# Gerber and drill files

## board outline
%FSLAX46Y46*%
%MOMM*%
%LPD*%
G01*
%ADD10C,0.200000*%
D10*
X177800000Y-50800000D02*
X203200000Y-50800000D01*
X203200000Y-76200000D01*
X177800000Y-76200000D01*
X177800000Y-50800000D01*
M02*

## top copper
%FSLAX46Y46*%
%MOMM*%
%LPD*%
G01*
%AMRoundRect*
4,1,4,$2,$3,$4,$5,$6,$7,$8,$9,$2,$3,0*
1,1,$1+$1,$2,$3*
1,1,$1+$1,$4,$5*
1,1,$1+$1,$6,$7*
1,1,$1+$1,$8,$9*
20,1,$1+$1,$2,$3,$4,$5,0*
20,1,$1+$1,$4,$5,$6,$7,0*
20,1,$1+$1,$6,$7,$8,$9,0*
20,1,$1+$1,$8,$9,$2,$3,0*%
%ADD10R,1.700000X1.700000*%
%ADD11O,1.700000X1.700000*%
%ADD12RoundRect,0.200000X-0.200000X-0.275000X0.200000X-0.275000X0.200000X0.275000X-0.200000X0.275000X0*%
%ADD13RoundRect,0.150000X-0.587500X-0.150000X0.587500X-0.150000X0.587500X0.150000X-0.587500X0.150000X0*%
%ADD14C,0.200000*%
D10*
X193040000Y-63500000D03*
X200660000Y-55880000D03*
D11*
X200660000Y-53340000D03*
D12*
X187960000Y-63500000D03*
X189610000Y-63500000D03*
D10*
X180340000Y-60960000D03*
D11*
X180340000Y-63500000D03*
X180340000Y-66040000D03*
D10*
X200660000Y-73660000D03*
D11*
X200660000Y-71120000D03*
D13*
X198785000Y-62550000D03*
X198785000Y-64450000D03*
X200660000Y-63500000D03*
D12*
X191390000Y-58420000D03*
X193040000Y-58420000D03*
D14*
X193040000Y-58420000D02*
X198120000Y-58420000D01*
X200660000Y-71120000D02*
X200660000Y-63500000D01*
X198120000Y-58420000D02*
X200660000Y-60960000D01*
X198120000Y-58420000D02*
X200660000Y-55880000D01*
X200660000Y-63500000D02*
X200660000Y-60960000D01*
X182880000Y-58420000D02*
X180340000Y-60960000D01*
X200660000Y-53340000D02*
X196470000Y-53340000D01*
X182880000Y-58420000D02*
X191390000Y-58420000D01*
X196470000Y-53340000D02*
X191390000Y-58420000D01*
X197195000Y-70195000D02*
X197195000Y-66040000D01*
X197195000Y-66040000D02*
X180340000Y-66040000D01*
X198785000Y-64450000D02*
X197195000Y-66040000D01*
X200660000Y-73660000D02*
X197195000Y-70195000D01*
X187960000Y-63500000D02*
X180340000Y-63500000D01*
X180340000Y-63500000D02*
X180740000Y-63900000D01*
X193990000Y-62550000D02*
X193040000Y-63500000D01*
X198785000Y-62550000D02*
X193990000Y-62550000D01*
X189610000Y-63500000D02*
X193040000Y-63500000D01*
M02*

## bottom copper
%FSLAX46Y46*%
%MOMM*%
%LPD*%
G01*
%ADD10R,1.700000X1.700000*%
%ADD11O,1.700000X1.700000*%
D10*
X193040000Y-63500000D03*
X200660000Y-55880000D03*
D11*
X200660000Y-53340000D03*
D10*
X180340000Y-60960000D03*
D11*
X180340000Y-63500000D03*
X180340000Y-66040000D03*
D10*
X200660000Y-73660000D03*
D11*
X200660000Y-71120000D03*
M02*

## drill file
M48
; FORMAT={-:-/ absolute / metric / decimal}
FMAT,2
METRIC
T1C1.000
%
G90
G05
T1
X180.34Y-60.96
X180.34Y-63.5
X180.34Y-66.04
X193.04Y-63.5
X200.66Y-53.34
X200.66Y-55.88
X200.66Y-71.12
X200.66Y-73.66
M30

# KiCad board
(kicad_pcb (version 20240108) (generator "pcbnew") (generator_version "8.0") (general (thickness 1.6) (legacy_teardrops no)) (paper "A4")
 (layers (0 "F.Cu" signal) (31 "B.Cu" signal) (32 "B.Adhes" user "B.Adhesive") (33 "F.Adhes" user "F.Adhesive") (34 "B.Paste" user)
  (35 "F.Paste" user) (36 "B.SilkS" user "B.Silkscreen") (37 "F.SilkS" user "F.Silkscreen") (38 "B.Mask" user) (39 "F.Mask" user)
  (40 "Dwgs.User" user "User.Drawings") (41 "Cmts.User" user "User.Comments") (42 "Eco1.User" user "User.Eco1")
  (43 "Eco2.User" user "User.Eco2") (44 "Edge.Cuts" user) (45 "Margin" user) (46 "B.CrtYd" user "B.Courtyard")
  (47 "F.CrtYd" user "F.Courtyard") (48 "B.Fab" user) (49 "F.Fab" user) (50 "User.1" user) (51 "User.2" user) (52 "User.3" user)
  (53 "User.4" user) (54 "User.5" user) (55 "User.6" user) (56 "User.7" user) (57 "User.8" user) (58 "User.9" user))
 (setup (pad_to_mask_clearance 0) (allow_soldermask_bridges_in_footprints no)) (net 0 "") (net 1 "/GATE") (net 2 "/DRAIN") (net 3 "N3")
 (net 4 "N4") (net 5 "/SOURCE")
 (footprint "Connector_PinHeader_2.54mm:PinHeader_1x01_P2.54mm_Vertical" (layer "F.Cu") (at 193.04 63.5)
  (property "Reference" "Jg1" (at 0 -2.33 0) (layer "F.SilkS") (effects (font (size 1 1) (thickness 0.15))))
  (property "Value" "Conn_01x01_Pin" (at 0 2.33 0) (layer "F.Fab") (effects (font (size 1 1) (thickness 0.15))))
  (pad "1" thru_hole rect (at 0 0) (size 1.7 1.7) (drill 1) (layers "*.Cu" "*.Mask") (remove_unused_layers no) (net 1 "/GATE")))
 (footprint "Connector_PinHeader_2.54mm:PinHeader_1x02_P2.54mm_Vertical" (layer "F.Cu") (at 200.66 55.88 180)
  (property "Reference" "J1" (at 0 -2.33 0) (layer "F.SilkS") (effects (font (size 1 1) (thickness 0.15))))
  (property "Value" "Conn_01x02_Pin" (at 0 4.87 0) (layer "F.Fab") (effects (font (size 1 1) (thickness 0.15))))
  (pad "1" thru_hole rect (at 0 0 180) (size 1.7 1.7) (drill 1) (layers "*.Cu" "*.Mask") (remove_unused_layers no) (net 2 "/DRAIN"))
  (pad "2" thru_hole oval (at 0 2.54 180) (size 1.7 1.7) (drill 1) (layers "*.Cu" "*.Mask") (remove_unused_layers no) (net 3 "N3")))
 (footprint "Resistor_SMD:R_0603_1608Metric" (layer "F.Cu") (at 188.785 63.5)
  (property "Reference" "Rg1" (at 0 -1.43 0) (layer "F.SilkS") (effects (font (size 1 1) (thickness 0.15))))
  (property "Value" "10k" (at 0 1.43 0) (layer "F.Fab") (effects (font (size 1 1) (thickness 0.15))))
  (pad "1" smd roundrect (at -0.825 0) (size 0.8 0.95) (layers "F.Cu" "F.Paste" "F.Mask") (roundrect_rratio 0.25) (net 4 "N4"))
  (pad "2" smd roundrect (at 0.825 0) (size 0.8 0.95) (layers "F.Cu" "F.Paste" "F.Mask") (roundrect_rratio 0.25) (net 1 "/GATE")))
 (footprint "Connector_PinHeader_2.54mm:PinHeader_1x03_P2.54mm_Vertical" (layer "F.Cu") (at 180.34 60.96)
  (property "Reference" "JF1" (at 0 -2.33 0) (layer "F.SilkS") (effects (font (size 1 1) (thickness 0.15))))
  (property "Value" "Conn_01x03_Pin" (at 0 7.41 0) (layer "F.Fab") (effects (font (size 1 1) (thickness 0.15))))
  (pad "1" thru_hole rect (at 0 0) (size 1.7 1.7) (drill 1) (layers "*.Cu" "*.Mask") (remove_unused_layers no) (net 3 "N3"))
  (pad "2" thru_hole oval (at 0 2.54) (size 1.7 1.7) (drill 1) (layers "*.Cu" "*.Mask") (remove_unused_layers no) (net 4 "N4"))
  (pad "3" thru_hole oval (at 0 5.08) (size 1.7 1.7) (drill 1) (layers "*.Cu" "*.Mask") (remove_unused_layers no) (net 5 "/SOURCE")))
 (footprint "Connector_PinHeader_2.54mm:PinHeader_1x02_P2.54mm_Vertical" (layer "F.Cu") (at 200.66 73.66 180)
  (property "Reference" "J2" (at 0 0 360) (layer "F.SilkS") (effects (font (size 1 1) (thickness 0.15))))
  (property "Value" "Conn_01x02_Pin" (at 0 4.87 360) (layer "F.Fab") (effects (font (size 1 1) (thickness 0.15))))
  (pad "1" thru_hole rect (at 0 0 180) (size 1.7 1.7) (drill 1) (layers "*.Cu" "*.Mask") (remove_unused_layers no) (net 5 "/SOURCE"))
  (pad "2" thru_hole oval (at 0 2.54 180) (size 1.7 1.7) (drill 1) (layers "*.Cu" "*.Mask") (remove_unused_layers no) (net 2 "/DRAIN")))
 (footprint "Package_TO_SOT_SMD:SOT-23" (layer "F.Cu") (at 199.7225 63.5)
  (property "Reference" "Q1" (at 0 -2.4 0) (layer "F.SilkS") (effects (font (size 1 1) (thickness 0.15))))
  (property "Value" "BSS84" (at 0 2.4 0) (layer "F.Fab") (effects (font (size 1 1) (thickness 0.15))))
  (pad "1" smd roundrect (at -0.9375 -0.95) (size 1.475 0.6) (layers "F.Cu" "F.Paste" "F.Mask") (roundrect_rratio 0.25) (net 1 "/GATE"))
  (pad "2" smd roundrect (at -0.9375 0.95) (size 1.475 0.6) (layers "F.Cu" "F.Paste" "F.Mask") (roundrect_rratio 0.25) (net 5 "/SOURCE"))
  (pad "3" smd roundrect (at 0.9375 0) (size 1.475 0.6) (layers "F.Cu" "F.Paste" "F.Mask") (roundrect_rratio 0.25) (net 2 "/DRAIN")))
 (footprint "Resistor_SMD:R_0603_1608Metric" (layer "F.Cu") (at 192.215 58.42)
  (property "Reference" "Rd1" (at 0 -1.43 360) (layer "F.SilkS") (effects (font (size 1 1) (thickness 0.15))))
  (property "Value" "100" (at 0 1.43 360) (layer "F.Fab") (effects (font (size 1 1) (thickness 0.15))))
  (pad "1" smd roundrect (at -0.825 0) (size 0.8 0.95) (layers "F.Cu" "F.Paste" "F.Mask") (roundrect_rratio 0.25) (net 3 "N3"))
  (pad "2" smd roundrect (at 0.825 0) (size 0.8 0.95) (layers "F.Cu" "F.Paste" "F.Mask") (roundrect_rratio 0.25) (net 2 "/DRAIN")))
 (gr_rect (start 177.8 50.8) (end 203.2 76.2) (stroke (width 0.2) (type default)) (fill none) (layer "Edge.Cuts"))
 (segment (start 193.04 58.42) (end 198.12 58.42) (width 0.2) (layer "F.Cu") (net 2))
 (segment (start 200.66 71.12) (end 200.66 63.5) (width 0.2) (layer "F.Cu") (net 2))
 (segment (start 198.12 58.42) (end 200.66 60.96) (width 0.2) (layer "F.Cu") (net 2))
 (segment (start 198.12 58.42) (end 200.66 55.88) (width 0.2) (layer "F.Cu") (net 2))
 (segment (start 200.66 63.5) (end 200.66 60.96) (width 0.2) (layer "F.Cu") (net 2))
 (segment (start 182.88 58.42) (end 180.34 60.96) (width 0.2) (layer "F.Cu") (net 3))
 (segment (start 200.66 53.34) (end 196.47 53.34) (width 0.2) (layer "F.Cu") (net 3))
 (segment (start 182.88 58.42) (end 191.39 58.42) (width 0.2) (layer "F.Cu") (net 3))
 (segment (start 196.47 53.34) (end 191.39 58.42) (width 0.2) (layer "F.Cu") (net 3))
 (segment (start 197.195 70.195) (end 197.195 66.04) (width 0.2) (layer "F.Cu") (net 5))
 (segment (start 197.195 66.04) (end 180.34 66.04) (width 0.2) (layer "F.Cu") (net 5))
 (segment (start 198.785 64.45) (end 197.195 66.04) (width 0.2) (layer "F.Cu") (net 5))
 (segment (start 200.66 73.66) (end 197.195 70.195) (width 0.2) (layer "F.Cu") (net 5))
 (segment (start 187.96 63.5) (end 180.34 63.5) (width 0.2) (layer "F.Cu") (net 4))
 (segment (start 180.34 63.5) (end 180.74 63.9) (width 0.2) (layer "F.Cu") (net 4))
 (segment (start 193.99 62.55) (end 193.04 63.5) (width 0.2) (layer "F.Cu") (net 1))
 (segment (start 198.785 62.55) (end 193.99 62.55) (width 0.2) (layer "F.Cu") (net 1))
 (segment (start 189.61 63.5) (end 193.04 63.5) (width 0.2) (layer "F.Cu") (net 1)))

